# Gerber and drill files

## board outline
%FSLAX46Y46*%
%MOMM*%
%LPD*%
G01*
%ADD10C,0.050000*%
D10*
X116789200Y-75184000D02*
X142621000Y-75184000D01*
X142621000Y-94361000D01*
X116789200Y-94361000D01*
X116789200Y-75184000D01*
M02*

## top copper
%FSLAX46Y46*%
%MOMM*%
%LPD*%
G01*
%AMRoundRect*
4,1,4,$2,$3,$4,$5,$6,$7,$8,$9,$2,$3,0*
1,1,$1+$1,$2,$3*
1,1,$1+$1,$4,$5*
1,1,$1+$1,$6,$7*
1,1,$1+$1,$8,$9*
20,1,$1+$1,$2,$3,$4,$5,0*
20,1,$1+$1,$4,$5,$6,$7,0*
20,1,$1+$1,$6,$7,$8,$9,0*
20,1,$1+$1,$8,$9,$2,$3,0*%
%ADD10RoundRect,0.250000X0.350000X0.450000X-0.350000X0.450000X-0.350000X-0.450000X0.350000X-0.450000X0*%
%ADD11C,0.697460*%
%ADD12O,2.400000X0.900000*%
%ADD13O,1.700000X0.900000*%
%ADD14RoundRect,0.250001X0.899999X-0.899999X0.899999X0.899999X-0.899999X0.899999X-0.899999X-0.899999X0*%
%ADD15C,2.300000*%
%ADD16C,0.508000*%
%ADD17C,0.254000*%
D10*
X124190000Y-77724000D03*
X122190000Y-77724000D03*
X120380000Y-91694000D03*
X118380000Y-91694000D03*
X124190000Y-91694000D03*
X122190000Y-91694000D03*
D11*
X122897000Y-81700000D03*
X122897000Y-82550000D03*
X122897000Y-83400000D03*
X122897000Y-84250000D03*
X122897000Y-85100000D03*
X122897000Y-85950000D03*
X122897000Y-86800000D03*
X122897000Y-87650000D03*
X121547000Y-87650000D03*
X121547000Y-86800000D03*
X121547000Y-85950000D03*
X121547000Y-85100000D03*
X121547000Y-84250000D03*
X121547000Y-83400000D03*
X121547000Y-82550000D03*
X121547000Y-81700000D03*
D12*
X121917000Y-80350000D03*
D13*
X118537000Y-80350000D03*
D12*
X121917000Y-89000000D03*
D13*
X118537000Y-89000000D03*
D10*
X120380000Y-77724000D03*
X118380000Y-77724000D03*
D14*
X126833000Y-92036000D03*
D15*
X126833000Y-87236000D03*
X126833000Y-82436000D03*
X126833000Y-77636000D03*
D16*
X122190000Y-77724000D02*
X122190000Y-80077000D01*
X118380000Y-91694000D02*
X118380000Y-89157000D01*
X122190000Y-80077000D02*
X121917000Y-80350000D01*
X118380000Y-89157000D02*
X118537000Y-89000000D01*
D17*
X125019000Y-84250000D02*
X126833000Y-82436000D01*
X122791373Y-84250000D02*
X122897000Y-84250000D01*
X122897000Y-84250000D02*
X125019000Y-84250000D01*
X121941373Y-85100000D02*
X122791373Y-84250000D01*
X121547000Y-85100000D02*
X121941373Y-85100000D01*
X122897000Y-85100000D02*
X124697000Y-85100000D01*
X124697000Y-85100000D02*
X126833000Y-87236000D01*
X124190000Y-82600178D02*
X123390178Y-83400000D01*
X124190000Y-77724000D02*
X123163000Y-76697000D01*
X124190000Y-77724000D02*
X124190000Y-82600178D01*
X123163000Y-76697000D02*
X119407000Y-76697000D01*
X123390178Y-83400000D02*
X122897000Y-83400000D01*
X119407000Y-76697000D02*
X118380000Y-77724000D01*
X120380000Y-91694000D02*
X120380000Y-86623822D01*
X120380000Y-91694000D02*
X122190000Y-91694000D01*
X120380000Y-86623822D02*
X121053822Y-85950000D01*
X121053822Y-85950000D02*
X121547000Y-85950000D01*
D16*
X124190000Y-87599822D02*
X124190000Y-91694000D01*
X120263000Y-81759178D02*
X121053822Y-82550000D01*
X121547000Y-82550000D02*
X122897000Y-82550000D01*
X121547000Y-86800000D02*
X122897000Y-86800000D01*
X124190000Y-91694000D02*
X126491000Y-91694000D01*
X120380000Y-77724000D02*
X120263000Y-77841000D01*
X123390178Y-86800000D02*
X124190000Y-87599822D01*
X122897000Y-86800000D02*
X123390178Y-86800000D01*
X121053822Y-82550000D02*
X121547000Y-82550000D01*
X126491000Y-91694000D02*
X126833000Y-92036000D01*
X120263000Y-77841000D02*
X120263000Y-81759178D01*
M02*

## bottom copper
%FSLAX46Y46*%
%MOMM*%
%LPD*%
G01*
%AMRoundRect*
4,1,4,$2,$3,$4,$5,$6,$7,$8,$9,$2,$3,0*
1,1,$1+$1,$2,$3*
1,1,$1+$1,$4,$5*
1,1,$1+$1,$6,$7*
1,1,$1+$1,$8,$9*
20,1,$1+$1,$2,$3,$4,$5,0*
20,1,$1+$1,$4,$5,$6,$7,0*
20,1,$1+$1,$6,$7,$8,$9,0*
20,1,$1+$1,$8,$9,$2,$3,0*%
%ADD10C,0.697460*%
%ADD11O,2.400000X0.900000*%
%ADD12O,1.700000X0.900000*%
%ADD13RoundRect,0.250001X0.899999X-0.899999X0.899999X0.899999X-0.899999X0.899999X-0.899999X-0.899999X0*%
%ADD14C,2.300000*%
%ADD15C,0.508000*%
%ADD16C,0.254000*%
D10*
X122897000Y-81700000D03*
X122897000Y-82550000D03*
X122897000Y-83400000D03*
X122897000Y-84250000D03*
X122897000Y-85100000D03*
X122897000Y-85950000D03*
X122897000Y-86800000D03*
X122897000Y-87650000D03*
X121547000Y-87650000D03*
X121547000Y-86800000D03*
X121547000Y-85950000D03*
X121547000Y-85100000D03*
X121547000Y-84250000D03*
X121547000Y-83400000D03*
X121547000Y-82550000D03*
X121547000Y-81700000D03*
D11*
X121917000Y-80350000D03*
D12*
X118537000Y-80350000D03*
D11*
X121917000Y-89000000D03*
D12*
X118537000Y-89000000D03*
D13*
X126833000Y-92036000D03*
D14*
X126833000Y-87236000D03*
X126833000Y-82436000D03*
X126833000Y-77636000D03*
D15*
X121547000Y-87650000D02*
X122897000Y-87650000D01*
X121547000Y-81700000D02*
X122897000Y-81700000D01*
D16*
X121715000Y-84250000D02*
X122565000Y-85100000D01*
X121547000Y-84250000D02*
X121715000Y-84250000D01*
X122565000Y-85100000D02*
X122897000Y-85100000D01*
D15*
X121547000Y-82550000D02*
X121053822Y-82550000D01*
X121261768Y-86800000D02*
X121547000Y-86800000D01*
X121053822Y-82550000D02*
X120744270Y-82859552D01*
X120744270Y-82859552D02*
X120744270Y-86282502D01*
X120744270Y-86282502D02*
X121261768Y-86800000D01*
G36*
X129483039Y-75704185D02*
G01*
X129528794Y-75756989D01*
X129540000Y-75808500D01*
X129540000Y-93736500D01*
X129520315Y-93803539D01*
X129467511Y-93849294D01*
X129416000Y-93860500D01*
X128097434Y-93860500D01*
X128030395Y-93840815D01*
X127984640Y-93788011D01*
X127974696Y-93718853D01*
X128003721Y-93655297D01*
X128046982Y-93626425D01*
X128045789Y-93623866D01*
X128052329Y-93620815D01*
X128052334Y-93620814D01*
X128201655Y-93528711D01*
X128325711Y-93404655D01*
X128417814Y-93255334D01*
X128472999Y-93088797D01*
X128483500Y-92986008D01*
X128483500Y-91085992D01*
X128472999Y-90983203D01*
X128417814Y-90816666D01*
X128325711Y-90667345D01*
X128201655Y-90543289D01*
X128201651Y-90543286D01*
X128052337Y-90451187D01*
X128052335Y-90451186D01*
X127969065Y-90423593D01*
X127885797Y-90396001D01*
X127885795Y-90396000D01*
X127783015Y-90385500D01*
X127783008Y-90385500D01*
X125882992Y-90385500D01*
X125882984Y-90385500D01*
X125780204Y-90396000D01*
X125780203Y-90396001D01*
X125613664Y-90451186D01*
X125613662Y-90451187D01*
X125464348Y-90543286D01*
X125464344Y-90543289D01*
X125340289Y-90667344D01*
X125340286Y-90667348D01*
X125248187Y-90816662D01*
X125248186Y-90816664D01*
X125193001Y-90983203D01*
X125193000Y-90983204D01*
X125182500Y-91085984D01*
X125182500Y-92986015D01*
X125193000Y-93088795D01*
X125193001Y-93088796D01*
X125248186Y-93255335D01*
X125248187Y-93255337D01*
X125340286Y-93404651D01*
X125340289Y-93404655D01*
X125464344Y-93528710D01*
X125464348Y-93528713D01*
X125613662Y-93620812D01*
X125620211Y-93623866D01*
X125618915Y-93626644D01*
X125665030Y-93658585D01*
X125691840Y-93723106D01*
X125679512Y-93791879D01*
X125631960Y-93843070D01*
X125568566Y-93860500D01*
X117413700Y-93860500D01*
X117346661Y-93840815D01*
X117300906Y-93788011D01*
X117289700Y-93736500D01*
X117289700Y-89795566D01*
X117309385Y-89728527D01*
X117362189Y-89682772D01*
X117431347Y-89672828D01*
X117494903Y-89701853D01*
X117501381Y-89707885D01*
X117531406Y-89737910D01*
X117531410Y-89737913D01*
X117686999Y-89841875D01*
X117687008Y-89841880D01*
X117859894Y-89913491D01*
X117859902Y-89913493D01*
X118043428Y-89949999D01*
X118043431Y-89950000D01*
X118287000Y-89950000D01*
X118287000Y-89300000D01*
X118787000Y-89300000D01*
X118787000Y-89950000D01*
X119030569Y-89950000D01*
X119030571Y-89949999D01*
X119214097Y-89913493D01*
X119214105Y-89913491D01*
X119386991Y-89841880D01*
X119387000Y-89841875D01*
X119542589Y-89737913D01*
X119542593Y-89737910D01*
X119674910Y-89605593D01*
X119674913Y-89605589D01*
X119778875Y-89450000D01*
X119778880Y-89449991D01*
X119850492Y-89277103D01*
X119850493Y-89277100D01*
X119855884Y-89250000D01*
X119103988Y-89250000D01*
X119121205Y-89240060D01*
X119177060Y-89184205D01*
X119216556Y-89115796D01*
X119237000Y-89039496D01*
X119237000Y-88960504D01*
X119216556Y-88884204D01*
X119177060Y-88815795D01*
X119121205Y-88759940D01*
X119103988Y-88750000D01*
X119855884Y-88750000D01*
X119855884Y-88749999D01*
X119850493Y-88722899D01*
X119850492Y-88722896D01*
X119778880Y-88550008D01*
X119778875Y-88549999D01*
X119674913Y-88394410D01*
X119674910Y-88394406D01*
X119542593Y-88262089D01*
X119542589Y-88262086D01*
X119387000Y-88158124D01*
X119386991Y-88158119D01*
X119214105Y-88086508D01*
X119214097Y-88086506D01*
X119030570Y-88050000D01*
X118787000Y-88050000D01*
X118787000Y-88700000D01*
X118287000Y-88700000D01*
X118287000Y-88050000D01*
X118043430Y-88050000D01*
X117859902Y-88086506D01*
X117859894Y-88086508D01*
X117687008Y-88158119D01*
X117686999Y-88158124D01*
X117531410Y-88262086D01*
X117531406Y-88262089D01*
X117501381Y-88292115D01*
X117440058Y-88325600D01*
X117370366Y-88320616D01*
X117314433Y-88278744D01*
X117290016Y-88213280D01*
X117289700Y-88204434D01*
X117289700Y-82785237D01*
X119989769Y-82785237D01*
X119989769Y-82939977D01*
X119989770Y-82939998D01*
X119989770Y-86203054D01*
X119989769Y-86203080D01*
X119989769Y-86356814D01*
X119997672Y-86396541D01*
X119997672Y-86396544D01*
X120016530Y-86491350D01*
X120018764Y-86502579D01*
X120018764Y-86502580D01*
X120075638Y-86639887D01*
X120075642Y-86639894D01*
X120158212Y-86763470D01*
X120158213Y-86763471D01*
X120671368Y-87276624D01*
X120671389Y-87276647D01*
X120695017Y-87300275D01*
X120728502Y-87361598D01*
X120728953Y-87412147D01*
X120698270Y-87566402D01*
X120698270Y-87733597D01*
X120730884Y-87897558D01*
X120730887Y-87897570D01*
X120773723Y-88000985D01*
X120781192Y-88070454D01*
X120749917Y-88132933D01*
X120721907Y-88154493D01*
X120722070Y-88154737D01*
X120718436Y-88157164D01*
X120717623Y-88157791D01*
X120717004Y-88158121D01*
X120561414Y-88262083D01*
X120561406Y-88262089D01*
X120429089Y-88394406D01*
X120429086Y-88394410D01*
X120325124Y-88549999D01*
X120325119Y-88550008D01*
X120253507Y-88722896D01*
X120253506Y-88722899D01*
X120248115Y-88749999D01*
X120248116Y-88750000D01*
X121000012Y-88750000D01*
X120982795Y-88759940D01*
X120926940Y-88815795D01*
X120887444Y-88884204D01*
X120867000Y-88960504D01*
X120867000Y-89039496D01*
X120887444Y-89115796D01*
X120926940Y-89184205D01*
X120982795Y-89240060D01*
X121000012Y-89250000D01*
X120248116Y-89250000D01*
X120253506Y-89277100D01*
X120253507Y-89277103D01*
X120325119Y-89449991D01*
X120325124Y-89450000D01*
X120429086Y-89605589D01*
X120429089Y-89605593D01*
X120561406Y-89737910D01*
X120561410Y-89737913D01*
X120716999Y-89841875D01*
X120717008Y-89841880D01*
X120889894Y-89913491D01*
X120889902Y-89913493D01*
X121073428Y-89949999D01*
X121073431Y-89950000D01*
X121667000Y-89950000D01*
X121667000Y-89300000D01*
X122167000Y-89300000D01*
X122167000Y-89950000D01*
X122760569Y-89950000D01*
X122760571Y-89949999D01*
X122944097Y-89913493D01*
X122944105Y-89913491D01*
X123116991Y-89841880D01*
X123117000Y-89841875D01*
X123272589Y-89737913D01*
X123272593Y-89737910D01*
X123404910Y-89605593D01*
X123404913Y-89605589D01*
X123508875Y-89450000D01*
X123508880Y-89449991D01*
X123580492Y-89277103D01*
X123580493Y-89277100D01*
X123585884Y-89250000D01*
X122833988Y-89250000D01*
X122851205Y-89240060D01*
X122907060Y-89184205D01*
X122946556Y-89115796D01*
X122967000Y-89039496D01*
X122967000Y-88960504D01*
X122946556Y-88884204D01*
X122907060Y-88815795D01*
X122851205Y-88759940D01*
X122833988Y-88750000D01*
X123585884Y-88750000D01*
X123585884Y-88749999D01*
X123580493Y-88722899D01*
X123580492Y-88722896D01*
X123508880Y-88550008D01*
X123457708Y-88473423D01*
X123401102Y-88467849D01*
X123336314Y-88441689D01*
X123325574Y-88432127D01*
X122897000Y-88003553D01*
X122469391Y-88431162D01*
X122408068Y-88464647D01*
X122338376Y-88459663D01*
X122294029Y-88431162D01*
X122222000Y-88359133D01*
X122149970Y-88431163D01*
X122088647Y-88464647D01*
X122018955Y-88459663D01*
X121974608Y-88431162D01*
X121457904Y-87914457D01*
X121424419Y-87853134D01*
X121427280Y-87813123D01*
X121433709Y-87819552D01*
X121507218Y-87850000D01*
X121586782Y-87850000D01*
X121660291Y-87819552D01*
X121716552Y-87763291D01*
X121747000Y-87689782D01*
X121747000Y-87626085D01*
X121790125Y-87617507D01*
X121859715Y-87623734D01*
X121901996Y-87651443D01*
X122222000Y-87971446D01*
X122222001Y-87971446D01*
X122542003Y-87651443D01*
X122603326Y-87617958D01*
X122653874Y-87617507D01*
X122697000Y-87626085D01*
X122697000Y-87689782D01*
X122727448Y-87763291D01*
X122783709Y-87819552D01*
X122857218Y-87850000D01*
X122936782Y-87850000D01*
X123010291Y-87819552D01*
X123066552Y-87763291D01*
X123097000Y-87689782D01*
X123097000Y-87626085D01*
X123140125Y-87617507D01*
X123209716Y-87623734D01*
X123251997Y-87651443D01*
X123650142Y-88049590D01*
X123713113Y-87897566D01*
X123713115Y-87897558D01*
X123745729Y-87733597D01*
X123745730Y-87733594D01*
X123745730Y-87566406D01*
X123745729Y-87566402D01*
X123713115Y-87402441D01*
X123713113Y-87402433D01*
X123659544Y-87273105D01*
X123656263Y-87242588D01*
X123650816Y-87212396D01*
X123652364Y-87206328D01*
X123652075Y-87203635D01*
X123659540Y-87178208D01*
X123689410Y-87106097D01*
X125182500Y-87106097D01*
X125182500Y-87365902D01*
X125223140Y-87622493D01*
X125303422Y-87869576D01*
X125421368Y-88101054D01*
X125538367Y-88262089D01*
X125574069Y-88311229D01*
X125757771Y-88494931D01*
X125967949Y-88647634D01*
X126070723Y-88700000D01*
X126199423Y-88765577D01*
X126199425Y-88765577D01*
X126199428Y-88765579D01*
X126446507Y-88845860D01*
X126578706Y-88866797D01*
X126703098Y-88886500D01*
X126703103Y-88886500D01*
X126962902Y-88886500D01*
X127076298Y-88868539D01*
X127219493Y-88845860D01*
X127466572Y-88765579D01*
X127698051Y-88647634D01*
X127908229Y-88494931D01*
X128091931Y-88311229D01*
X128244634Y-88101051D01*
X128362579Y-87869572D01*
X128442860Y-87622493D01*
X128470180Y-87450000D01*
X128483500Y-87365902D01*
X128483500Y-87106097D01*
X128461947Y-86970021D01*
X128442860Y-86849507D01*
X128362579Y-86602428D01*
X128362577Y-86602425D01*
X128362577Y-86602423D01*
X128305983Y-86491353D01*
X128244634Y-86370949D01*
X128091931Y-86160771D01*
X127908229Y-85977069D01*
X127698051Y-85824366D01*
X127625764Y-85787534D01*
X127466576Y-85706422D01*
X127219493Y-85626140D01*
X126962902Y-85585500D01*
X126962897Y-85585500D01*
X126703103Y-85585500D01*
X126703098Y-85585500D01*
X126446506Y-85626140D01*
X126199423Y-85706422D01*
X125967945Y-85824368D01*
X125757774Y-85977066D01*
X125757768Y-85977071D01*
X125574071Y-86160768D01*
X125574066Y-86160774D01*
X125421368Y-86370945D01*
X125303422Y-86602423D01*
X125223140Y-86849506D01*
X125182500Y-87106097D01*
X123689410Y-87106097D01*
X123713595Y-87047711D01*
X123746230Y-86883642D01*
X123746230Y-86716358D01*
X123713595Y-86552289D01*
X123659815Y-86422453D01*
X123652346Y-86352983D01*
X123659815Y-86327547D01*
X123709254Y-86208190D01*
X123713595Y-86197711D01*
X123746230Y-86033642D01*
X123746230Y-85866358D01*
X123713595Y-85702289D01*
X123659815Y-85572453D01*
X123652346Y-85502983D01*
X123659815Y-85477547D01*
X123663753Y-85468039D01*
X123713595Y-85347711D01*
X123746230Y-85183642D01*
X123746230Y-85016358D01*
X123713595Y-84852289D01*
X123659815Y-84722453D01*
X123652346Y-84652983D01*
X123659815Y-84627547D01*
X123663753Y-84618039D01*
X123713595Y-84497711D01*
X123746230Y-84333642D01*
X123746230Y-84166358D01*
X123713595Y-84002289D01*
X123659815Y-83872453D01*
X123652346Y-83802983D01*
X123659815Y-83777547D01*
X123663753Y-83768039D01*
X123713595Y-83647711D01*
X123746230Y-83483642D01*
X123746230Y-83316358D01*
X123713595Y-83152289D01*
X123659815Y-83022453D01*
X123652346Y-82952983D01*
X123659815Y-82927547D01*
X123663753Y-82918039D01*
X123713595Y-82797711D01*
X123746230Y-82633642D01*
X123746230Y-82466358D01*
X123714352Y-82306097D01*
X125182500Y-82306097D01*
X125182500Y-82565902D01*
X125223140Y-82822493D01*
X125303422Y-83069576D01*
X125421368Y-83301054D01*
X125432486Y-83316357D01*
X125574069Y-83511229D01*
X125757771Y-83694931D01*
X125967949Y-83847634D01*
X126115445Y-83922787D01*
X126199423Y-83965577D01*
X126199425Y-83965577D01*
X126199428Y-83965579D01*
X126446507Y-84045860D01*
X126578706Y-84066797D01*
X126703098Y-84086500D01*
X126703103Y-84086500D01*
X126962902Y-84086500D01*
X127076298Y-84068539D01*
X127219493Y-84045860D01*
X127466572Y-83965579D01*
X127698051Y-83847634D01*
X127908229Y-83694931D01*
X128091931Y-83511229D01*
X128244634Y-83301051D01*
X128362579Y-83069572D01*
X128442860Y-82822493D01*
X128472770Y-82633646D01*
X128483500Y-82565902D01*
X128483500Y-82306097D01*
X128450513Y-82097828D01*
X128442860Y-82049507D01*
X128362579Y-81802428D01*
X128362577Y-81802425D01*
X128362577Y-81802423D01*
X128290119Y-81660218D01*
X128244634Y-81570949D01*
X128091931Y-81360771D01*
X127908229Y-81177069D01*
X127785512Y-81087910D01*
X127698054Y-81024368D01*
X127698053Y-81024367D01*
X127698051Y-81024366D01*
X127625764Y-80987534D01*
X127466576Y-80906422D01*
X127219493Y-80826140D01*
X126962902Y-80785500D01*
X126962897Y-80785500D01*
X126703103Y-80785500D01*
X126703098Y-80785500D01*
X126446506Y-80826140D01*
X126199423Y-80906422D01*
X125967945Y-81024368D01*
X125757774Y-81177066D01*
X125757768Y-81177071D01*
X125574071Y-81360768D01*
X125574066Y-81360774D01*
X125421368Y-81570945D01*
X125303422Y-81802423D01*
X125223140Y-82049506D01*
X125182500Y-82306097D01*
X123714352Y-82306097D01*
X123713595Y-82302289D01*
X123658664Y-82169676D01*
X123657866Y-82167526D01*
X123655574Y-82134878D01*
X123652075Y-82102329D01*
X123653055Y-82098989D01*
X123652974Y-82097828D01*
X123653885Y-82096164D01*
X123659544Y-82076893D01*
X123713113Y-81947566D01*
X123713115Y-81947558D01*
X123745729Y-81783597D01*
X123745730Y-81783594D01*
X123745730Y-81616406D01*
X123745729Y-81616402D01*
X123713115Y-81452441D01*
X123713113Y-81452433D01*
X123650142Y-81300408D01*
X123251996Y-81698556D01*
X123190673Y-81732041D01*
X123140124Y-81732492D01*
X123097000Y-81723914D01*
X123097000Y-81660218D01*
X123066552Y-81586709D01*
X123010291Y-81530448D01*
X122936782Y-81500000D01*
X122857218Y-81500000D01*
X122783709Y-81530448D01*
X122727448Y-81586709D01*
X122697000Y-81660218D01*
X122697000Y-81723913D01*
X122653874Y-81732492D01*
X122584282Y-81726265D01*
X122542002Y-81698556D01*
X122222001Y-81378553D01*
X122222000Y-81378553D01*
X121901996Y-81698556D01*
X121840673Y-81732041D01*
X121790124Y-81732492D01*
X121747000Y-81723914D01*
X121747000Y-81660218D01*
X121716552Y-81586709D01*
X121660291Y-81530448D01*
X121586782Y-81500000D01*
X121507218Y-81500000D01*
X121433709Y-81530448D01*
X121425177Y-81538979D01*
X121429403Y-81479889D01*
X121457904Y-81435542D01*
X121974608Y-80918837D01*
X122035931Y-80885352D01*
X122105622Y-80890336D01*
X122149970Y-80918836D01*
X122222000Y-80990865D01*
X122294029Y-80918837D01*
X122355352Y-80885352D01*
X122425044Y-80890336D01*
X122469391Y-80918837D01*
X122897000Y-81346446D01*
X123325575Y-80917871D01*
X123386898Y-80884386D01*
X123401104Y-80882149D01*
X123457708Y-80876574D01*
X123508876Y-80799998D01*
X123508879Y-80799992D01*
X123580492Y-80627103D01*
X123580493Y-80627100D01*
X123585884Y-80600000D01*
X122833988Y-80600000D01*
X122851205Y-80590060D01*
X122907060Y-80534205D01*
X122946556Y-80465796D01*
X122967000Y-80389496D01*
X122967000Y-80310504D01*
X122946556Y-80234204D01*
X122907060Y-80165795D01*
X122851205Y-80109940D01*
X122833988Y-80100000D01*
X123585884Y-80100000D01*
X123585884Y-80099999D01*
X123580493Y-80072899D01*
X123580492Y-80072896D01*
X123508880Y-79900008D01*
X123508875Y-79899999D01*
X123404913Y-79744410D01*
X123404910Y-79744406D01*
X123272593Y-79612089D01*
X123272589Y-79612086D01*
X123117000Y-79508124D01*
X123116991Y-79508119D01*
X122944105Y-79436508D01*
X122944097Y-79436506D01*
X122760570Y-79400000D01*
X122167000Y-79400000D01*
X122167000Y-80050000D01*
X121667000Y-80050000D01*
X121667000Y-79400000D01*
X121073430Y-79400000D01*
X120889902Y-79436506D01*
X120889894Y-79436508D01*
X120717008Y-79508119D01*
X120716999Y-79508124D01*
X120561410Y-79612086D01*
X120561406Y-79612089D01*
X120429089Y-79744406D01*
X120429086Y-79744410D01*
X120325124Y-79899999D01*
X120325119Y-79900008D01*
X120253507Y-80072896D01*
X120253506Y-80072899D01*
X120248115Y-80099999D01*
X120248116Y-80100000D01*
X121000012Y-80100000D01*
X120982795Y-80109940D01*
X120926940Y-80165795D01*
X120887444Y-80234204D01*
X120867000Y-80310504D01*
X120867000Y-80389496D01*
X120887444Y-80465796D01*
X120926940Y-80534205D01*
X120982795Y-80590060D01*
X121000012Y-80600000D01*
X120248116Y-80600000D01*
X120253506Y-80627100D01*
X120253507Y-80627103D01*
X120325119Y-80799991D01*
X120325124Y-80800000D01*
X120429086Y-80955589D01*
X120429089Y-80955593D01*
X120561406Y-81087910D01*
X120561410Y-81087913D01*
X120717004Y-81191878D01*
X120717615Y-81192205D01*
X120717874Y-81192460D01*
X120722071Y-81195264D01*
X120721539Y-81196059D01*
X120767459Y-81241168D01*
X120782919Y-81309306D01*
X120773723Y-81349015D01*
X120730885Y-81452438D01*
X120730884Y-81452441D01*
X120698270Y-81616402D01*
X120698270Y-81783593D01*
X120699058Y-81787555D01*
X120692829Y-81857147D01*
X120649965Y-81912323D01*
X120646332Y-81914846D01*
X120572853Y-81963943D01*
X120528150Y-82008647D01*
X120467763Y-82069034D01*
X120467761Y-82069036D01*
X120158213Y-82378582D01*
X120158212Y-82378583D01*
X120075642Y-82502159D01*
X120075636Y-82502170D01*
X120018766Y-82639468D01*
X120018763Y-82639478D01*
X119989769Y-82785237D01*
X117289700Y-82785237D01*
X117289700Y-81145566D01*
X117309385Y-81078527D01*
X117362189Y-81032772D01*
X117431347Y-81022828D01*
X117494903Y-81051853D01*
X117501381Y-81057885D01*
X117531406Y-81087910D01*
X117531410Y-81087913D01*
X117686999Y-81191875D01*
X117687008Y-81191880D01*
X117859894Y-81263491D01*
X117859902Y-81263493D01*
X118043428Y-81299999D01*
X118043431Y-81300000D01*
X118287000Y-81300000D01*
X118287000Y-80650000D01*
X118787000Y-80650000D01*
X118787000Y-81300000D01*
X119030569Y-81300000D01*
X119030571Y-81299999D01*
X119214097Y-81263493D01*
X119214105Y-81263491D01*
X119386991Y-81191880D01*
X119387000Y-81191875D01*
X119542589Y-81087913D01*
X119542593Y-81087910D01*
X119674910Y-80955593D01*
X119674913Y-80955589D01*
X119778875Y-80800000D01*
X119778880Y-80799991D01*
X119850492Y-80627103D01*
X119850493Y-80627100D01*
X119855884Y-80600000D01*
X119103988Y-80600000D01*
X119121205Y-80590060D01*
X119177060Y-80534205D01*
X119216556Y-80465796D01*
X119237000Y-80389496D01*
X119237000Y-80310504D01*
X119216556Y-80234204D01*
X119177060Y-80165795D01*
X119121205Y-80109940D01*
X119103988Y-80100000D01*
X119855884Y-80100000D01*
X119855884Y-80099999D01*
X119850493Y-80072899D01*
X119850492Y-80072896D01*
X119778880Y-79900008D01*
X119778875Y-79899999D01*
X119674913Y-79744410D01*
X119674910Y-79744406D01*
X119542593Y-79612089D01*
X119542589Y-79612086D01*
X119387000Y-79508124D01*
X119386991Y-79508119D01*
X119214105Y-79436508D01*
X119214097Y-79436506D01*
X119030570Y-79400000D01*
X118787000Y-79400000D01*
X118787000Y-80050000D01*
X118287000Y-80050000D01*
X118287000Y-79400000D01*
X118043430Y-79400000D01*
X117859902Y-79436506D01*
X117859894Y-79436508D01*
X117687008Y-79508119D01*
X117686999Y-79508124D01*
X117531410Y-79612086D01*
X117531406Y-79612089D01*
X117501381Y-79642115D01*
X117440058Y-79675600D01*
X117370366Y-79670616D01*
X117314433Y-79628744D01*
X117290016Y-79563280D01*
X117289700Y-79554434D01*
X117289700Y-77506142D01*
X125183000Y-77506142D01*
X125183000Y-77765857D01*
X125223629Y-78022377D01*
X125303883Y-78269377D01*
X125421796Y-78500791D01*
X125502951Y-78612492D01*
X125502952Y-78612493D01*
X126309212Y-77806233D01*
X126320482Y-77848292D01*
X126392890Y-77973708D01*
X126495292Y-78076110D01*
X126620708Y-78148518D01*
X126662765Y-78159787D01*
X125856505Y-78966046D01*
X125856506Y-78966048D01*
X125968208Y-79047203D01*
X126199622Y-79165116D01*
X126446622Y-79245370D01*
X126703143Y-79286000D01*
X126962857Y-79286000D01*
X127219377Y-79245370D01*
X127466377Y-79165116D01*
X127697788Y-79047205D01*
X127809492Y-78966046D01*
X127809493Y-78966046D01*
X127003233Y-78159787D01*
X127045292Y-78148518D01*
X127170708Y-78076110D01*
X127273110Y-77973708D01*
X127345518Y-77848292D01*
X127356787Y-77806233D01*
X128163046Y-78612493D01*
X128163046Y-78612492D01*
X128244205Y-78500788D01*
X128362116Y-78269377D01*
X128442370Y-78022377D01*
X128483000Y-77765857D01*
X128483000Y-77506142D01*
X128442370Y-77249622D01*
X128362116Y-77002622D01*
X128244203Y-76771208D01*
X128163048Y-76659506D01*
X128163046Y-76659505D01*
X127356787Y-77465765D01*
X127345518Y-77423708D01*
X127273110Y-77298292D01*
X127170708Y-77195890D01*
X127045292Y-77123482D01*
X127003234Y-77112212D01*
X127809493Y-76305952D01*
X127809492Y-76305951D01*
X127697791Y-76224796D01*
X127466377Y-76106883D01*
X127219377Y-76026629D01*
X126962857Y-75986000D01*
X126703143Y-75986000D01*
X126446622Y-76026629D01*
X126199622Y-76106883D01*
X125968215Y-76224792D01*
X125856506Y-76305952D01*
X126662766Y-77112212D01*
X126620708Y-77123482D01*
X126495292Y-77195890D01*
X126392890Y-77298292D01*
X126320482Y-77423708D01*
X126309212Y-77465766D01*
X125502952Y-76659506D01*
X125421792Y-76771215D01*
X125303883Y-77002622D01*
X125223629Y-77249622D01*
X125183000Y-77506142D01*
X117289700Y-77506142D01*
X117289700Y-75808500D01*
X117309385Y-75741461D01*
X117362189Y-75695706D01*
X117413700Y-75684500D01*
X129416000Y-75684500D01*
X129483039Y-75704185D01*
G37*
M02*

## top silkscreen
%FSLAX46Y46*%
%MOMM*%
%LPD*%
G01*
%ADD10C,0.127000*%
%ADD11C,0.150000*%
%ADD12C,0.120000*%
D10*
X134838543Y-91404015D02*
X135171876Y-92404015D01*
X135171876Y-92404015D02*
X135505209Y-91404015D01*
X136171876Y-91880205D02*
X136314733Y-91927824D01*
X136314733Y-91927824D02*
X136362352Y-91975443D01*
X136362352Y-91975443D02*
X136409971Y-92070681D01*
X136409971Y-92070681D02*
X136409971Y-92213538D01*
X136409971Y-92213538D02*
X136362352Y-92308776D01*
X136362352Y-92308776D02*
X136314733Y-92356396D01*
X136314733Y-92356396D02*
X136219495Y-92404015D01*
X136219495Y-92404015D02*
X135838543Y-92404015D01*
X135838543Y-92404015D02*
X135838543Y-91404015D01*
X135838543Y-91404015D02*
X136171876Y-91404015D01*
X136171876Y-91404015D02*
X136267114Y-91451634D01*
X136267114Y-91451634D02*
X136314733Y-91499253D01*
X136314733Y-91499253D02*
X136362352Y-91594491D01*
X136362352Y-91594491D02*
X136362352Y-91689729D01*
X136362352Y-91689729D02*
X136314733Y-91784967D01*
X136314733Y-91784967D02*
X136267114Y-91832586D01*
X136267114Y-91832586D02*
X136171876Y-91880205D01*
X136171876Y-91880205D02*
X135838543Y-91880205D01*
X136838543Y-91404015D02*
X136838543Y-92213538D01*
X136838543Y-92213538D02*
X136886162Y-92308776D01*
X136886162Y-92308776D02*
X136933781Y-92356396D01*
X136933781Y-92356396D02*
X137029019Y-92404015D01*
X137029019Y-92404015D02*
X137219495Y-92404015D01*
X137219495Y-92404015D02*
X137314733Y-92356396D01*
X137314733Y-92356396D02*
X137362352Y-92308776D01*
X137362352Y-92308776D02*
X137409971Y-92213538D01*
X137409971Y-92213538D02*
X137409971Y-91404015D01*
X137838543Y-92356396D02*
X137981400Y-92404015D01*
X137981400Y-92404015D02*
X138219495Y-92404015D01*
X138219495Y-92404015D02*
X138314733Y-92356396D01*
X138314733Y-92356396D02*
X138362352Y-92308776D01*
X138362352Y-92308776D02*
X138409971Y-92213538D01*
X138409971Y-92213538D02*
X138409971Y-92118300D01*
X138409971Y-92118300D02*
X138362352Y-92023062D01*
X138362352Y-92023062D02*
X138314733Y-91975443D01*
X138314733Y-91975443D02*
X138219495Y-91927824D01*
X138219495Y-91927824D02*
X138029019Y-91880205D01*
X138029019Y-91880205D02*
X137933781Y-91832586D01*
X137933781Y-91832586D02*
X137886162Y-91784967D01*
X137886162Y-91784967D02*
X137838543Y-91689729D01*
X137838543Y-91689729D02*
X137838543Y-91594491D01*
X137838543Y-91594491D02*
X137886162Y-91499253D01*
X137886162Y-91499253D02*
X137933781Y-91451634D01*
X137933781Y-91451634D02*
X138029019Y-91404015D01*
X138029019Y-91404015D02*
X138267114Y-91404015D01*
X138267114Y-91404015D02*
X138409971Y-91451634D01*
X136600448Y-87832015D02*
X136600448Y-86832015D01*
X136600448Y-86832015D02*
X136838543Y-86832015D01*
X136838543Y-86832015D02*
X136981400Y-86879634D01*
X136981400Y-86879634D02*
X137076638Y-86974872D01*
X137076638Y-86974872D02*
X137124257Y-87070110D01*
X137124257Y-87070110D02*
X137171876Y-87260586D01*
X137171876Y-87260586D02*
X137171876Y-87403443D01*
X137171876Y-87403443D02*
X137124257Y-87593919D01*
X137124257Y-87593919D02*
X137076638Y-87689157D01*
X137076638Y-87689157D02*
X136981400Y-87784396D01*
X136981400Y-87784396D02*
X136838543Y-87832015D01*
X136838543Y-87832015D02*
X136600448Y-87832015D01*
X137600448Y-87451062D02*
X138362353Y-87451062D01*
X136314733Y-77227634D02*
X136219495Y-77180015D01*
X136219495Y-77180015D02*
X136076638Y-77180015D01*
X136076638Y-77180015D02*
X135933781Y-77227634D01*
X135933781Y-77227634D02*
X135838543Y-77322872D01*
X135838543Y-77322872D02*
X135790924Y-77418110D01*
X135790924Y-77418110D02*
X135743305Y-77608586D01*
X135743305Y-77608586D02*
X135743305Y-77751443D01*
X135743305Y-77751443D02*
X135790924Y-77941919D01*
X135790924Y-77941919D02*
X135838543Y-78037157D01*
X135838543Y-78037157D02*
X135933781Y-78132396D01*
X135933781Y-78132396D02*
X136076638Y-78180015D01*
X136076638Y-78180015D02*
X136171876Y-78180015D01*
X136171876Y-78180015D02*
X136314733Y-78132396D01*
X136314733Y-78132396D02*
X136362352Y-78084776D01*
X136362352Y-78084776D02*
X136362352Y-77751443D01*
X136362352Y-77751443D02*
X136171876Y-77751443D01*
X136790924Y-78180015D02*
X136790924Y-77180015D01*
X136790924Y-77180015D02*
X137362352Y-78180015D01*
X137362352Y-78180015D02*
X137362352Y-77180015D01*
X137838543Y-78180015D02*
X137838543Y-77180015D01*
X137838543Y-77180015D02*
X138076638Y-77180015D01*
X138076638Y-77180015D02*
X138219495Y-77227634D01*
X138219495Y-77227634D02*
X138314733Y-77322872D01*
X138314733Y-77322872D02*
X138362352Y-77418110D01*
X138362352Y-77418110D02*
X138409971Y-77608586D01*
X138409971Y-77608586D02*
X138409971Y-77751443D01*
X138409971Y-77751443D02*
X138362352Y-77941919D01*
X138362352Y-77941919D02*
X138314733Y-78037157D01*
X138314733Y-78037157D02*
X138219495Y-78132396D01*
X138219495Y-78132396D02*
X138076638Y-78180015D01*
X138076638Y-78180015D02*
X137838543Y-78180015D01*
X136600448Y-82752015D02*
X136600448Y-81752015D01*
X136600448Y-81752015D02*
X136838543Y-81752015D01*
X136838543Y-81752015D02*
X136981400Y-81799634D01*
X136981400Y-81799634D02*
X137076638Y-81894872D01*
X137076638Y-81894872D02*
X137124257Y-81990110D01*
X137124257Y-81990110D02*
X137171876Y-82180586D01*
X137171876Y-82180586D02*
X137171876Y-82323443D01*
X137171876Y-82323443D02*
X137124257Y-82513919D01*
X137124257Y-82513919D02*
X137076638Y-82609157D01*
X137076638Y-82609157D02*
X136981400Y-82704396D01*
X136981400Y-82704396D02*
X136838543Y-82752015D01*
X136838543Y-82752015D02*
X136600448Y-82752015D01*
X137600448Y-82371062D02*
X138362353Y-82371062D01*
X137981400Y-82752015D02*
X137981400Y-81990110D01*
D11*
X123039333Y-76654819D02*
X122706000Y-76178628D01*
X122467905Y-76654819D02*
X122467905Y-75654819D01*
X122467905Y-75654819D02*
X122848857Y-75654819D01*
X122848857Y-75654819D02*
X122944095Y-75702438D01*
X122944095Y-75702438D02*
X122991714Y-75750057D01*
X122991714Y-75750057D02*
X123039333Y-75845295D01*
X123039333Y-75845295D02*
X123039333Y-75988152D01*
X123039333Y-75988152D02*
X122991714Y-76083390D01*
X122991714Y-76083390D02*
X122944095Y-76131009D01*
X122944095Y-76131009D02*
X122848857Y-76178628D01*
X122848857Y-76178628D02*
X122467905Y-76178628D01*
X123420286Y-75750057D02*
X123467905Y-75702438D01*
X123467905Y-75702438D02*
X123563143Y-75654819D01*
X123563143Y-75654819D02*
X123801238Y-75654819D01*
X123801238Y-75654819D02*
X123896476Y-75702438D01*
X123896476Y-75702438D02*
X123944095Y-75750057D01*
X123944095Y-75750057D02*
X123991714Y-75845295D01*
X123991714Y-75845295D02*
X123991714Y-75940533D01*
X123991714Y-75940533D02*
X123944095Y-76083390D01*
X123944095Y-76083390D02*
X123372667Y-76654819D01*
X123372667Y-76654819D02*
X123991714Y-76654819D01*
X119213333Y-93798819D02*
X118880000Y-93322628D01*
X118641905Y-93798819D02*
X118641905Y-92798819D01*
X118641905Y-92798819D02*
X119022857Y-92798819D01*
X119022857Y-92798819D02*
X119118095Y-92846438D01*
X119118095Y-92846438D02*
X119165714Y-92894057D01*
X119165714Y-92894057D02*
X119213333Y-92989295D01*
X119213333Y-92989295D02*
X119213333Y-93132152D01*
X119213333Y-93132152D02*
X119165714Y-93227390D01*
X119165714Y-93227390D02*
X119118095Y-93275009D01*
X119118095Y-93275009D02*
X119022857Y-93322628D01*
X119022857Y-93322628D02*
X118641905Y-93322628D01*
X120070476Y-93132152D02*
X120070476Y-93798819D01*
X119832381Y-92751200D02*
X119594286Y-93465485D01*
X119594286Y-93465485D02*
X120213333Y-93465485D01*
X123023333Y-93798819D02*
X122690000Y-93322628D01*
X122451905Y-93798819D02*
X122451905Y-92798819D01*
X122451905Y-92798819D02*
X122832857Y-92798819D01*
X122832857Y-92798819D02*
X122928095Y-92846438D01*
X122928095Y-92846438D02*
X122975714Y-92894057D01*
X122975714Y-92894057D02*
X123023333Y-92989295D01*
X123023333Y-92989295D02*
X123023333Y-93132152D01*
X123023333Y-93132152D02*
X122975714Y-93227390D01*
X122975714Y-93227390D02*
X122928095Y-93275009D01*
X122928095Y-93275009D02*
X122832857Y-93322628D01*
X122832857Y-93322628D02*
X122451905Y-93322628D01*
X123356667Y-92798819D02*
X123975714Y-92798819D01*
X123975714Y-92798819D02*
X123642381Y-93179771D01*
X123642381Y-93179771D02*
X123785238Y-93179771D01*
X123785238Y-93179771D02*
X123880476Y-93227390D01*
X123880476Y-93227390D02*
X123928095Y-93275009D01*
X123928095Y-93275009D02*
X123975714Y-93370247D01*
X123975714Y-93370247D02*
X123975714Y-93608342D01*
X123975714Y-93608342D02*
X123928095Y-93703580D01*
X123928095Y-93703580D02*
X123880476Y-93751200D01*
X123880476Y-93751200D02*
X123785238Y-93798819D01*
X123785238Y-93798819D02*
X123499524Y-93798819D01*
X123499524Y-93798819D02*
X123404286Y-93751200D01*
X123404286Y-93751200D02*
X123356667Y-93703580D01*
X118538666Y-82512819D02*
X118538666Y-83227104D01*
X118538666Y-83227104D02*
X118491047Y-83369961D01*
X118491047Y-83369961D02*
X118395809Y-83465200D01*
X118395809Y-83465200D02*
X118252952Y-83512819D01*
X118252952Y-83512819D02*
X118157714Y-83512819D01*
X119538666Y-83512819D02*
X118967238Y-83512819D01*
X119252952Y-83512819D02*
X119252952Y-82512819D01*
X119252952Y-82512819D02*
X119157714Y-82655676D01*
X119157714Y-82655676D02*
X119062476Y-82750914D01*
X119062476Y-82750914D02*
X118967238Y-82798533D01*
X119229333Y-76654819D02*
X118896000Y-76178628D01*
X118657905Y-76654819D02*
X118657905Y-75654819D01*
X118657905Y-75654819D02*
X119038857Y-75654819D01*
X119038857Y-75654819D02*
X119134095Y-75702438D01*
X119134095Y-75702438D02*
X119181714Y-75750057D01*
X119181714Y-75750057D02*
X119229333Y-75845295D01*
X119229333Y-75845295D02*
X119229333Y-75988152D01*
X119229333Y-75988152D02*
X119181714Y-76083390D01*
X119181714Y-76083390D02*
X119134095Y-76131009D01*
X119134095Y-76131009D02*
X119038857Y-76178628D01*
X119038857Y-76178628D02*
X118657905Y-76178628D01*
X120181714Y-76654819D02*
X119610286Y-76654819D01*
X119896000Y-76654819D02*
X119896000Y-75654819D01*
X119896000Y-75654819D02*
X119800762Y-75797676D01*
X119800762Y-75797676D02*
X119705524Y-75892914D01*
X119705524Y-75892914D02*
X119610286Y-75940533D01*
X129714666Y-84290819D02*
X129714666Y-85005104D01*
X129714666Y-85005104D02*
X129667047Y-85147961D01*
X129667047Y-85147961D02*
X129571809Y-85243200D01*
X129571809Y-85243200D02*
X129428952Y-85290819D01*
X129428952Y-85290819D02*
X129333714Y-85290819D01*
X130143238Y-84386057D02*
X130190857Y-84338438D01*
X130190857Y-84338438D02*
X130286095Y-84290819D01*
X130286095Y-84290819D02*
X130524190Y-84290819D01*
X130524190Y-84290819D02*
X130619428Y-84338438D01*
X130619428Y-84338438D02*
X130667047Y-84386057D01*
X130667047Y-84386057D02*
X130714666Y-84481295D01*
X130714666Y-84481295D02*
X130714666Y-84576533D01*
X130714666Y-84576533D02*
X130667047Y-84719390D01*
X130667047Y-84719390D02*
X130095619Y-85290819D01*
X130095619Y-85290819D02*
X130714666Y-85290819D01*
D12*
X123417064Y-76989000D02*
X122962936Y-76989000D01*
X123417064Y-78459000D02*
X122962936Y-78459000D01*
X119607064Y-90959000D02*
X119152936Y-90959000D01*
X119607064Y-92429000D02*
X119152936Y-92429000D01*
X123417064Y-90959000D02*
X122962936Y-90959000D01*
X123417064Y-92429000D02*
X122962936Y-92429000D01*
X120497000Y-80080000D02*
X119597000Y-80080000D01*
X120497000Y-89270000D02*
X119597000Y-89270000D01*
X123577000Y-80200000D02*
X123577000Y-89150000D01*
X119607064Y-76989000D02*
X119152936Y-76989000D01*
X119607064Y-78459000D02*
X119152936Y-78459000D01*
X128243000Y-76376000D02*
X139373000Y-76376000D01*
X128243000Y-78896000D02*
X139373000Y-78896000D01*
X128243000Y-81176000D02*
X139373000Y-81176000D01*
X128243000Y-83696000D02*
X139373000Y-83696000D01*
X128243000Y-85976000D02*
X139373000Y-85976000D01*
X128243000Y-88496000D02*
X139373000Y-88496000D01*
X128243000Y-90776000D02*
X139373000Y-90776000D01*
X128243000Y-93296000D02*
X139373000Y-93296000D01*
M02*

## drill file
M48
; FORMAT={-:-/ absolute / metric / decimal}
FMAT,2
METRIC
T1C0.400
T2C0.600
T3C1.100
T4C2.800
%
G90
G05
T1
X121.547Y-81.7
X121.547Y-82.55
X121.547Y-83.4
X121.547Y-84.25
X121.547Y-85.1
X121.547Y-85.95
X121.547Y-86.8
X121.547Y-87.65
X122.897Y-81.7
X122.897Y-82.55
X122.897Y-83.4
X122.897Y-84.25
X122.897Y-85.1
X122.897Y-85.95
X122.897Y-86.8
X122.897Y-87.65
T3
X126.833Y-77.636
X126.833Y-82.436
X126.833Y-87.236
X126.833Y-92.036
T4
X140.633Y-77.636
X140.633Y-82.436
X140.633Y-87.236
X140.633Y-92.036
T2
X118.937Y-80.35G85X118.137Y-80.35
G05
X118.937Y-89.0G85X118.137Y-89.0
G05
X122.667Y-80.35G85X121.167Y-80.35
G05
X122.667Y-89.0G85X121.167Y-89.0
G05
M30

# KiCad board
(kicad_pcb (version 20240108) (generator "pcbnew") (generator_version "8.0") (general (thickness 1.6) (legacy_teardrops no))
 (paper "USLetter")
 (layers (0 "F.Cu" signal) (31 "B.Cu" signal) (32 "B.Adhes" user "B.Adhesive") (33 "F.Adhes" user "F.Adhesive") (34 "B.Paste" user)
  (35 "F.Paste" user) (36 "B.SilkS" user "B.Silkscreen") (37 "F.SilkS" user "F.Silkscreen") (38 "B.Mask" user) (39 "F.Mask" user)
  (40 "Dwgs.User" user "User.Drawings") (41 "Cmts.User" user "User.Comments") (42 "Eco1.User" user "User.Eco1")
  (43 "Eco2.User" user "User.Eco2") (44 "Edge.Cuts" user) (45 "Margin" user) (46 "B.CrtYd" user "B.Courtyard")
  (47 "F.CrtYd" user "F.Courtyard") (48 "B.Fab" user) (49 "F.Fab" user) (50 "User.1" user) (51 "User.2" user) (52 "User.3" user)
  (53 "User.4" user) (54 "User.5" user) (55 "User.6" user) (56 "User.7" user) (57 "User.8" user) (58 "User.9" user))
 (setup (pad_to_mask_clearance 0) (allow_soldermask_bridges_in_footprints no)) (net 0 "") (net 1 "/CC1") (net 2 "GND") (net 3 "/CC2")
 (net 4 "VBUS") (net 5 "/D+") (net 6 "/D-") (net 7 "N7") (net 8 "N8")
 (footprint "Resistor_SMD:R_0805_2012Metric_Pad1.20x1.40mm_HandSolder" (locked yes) (layer "F.Cu") (at 123.19 77.724 180)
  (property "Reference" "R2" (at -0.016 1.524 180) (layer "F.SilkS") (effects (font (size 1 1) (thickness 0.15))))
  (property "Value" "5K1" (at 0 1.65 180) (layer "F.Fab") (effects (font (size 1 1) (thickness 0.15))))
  (fp_line (start -0.227064 0.735) (end 0.227064 0.735) (stroke (width 0.12) (type solid)) (layer "F.SilkS"))
  (fp_line (start -0.227064 -0.735) (end 0.227064 -0.735) (stroke (width 0.12) (type solid)) (layer "F.SilkS"))
  (pad "1" smd roundrect (at -1 0 180) (size 1.2 1.4) (layers "F.Cu" "F.Paste" "F.Mask") (roundrect_rratio 0.208333) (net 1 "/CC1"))
  (pad "2" smd roundrect (at 1 0 180) (size 1.2 1.4) (layers "F.Cu" "F.Paste" "F.Mask") (roundrect_rratio 0.208333) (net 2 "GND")))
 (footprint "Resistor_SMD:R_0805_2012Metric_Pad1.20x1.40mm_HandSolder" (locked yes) (layer "F.Cu") (at 119.38 91.694 180)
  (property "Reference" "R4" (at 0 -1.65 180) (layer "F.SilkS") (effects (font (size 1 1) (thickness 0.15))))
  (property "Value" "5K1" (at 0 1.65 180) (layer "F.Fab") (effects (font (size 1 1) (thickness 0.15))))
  (fp_line (start -0.227064 0.735) (end 0.227064 0.735) (stroke (width 0.12) (type solid)) (layer "F.SilkS"))
  (fp_line (start -0.227064 -0.735) (end 0.227064 -0.735) (stroke (width 0.12) (type solid)) (layer "F.SilkS"))
  (pad "1" smd roundrect (at -1 0 180) (size 1.2 1.4) (layers "F.Cu" "F.Paste" "F.Mask") (roundrect_rratio 0.208333) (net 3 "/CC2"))
  (pad "2" smd roundrect (at 1 0 180) (size 1.2 1.4) (layers "F.Cu" "F.Paste" "F.Mask") (roundrect_rratio 0.208333) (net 2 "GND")))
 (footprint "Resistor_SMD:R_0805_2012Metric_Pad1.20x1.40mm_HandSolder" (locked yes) (layer "F.Cu") (at 123.19 91.694 180)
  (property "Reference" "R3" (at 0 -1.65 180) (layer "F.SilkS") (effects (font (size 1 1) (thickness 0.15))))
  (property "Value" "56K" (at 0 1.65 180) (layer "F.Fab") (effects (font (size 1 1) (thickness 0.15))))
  (fp_line (start -0.227064 0.735) (end 0.227064 0.735) (stroke (width 0.12) (type solid)) (layer "F.SilkS"))
  (fp_line (start -0.227064 -0.735) (end 0.227064 -0.735) (stroke (width 0.12) (type solid)) (layer "F.SilkS"))
  (pad "1" smd roundrect (at -1 0 180) (size 1.2 1.4) (layers "F.Cu" "F.Paste" "F.Mask") (roundrect_rratio 0.208333) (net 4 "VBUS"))
  (pad "2" smd roundrect (at 1 0 180) (size 1.2 1.4) (layers "F.Cu" "F.Paste" "F.Mask") (roundrect_rratio 0.208333) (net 3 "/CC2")))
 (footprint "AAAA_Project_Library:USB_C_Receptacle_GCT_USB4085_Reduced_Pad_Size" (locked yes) (layer "F.Cu") (at 122.897 81.7 -90)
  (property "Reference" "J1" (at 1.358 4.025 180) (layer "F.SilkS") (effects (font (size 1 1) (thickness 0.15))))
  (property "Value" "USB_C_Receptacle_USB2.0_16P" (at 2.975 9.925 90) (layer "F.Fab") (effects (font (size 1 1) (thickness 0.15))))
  (fp_line (start -1.62 2.4) (end -1.62 3.3) (stroke (width 0.12) (type solid)) (layer "F.SilkS"))
  (fp_line (start 7.57 2.4) (end 7.57 3.3) (stroke (width 0.12) (type solid)) (layer "F.SilkS"))
  (fp_line (start -1.5 -0.68) (end 7.45 -0.68) (stroke (width 0.12) (type solid)) (layer "F.SilkS"))
  (pad "A1" thru_hole circle (at 0 0 270) (size 0.69746 0.69746) (drill 0.4) (layers "*.Cu" "*.Mask") (remove_unused_layers no)
   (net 2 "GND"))
  (pad "A4" thru_hole circle (at 0.85 0 270) (size 0.69746 0.69746) (drill 0.4) (layers "*.Cu" "*.Mask") (remove_unused_layers no)
   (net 4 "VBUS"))
  (pad "A5" thru_hole circle (at 1.7 0 270) (size 0.69746 0.69746) (drill 0.4) (layers "*.Cu" "*.Mask") (remove_unused_layers no)
   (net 1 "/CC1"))
  (pad "A6" thru_hole circle (at 2.55 0 270) (size 0.69746 0.69746) (drill 0.4) (layers "*.Cu" "*.Mask") (remove_unused_layers no)
   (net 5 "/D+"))
  (pad "A7" thru_hole circle (at 3.4 0 270) (size 0.69746 0.69746) (drill 0.4) (layers "*.Cu" "*.Mask") (remove_unused_layers no)
   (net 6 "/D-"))
  (pad "A8" thru_hole circle (at 4.25 0 270) (size 0.69746 0.69746) (drill 0.4) (layers "*.Cu" "*.Mask") (remove_unused_layers no)
   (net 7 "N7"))
  (pad "A9" thru_hole circle (at 5.1 0 270) (size 0.69746 0.69746) (drill 0.4) (layers "*.Cu" "*.Mask") (remove_unused_layers no)
   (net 4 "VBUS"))
  (pad "A12" thru_hole circle (at 5.95 0 270) (size 0.69746 0.69746) (drill 0.4) (layers "*.Cu" "*.Mask") (remove_unused_layers no)
   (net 2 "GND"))
  (pad "B1" thru_hole circle (at 5.95 1.35 270) (size 0.69746 0.69746) (drill 0.4) (layers "*.Cu" "*.Mask") (remove_unused_layers no)
   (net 2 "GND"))
  (pad "B4" thru_hole circle (at 5.1 1.35 270) (size 0.69746 0.69746) (drill 0.4) (layers "*.Cu" "*.Mask") (remove_unused_layers no)
   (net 4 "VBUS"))
  (pad "B5" thru_hole circle (at 4.25 1.35 270) (size 0.69746 0.69746) (drill 0.4) (layers "*.Cu" "*.Mask") (remove_unused_layers no)
   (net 3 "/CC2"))
  (pad "B6" thru_hole circle (at 3.4 1.35 270) (size 0.69746 0.69746) (drill 0.4) (layers "*.Cu" "*.Mask") (remove_unused_layers no)
   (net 5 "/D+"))
  (pad "B7" thru_hole circle (at 2.55 1.35 270) (size 0.69746 0.69746) (drill 0.4) (layers "*.Cu" "*.Mask") (remove_unused_layers no)
   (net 6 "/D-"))
  (pad "B8" thru_hole circle (at 1.7 1.35 270) (size 0.69746 0.69746) (drill 0.4) (layers "*.Cu" "*.Mask") (remove_unused_layers no)
   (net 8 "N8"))
  (pad "B9" thru_hole circle (at 0.85 1.35 270) (size 0.69746 0.69746) (drill 0.4) (layers "*.Cu" "*.Mask") (remove_unused_layers no)
   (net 4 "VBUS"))
  (pad "B12" thru_hole circle (at 0 1.35 270) (size 0.69746 0.69746) (drill 0.4) (layers "*.Cu" "*.Mask") (remove_unused_layers no)
   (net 2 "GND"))
  (pad "S1" thru_hole oval (at -1.35 0.98 270) (size 0.9 2.4) (drill oval 0.6 2.1) (layers "*.Cu" "*.Mask") (remove_unused_layers no)
   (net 2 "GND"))
  (pad "S1" thru_hole oval (at -1.35 4.36 270) (size 0.9 1.7) (drill oval 0.6 1.4) (layers "*.Cu" "*.Mask") (remove_unused_layers no)
   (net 2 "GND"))
  (pad "S1" thru_hole oval (at 7.3 0.98 270) (size 0.9 2.4) (drill oval 0.6 2.1) (layers "*.Cu" "*.Mask") (remove_unused_layers no)
   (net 2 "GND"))
  (pad "S1" thru_hole oval (at 7.3 4.36 270) (size 0.9 1.7) (drill oval 0.6 1.4) (layers "*.Cu" "*.Mask") (remove_unused_layers no)
   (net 2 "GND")))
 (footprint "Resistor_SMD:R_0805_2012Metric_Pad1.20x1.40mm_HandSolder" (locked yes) (layer "F.Cu") (at 119.38 77.724 180)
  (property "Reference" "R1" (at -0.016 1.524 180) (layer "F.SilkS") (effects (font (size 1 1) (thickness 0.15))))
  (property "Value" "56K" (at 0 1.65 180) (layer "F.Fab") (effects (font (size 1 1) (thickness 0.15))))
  (fp_line (start -0.227064 0.735) (end 0.227064 0.735) (stroke (width 0.12) (type solid)) (layer "F.SilkS"))
  (fp_line (start -0.227064 -0.735) (end 0.227064 -0.735) (stroke (width 0.12) (type solid)) (layer "F.SilkS"))
  (pad "1" smd roundrect (at -1 0 180) (size 1.2 1.4) (layers "F.Cu" "F.Paste" "F.Mask") (roundrect_rratio 0.208333) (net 4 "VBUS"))
  (pad "2" smd roundrect (at 1 0 180) (size 1.2 1.4) (layers "F.Cu" "F.Paste" "F.Mask") (roundrect_rratio 0.208333) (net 1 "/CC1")))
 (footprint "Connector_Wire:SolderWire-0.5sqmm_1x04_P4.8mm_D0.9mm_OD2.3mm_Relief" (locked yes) (layer "F.Cu") (at 126.833 92.036 90)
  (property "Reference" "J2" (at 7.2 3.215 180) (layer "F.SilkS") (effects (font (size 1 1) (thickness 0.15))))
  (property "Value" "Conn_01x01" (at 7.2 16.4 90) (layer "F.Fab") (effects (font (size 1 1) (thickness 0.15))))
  (fp_line (start 15.66 1.41) (end 15.66 12.54) (stroke (width 0.12) (type solid)) (layer "F.SilkS"))
  (fp_line (start 13.14 1.41) (end 13.14 12.54) (stroke (width 0.12) (type solid)) (layer "F.SilkS"))
  (fp_line (start 10.86 1.41) (end 10.86 12.54) (stroke (width 0.12) (type solid)) (layer "F.SilkS"))
  (fp_line (start 8.34 1.41) (end 8.34 12.54) (stroke (width 0.12) (type solid)) (layer "F.SilkS"))
  (fp_line (start 6.06 1.41) (end 6.06 12.54) (stroke (width 0.12) (type solid)) (layer "F.SilkS"))
  (fp_line (start 3.54 1.41) (end 3.54 12.54) (stroke (width 0.12) (type solid)) (layer "F.SilkS"))
  (fp_line (start 1.26 1.41) (end 1.26 12.54) (stroke (width 0.12) (type solid)) (layer "F.SilkS"))
  (fp_line (start -1.26 1.41) (end -1.26 12.54) (stroke (width 0.12) (type solid)) (layer "F.SilkS"))
  (pad "" np_thru_hole circle (at 0 13.8 90) (size 2.8 2.8) (drill 2.8) (layers "*.Cu" "*.Mask"))
  (pad "" np_thru_hole circle (at 4.8 13.8 90) (size 2.8 2.8) (drill 2.8) (layers "*.Cu" "*.Mask"))
  (pad "" np_thru_hole circle (at 9.6 13.8 90) (size 2.8 2.8) (drill 2.8) (layers "*.Cu" "*.Mask"))
  (pad "" np_thru_hole circle (at 14.4 13.8 90) (size 2.8 2.8) (drill 2.8) (layers "*.Cu" "*.Mask"))
  (pad "1" thru_hole roundrect (at 0 0 90) (size 2.3 2.3) (drill 1.1) (layers "*.Cu" "*.Mask") (remove_unused_layers no)
   (roundrect_rratio 0.108696) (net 4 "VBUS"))
  (pad "2" thru_hole circle (at 4.8 0 90) (size 2.3 2.3) (drill 1.1) (layers "*.Cu" "*.Mask") (remove_unused_layers no) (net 6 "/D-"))
  (pad "3" thru_hole circle (at 9.6 0 90) (size 2.3 2.3) (drill 1.1) (layers "*.Cu" "*.Mask") (remove_unused_layers no) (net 5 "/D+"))
  (pad "4" thru_hole circle (at 14.4 0 90) (size 2.3 2.3) (drill 1.1) (layers "*.Cu" "*.Mask") (remove_unused_layers no) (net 2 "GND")))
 (gr_rect (start 116.7892 75.184) (end 142.621 94.361) (locked yes) (stroke (width 0.05) (type default)) (fill none) (layer "Edge.Cuts"))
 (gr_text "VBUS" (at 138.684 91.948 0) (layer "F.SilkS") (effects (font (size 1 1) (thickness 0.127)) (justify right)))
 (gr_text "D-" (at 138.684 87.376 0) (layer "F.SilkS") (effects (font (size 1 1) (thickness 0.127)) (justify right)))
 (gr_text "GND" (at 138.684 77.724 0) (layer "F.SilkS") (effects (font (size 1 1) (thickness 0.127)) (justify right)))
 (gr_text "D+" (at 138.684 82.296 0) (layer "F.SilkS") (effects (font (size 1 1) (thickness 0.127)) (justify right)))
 (segment (start 122.19 77.724) (end 122.19 80.077) (width 0.508) (layer "F.Cu") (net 2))
 (segment (start 118.38 91.694) (end 118.38 89.157) (width 0.508) (layer "F.Cu") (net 2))
 (segment (start 122.19 80.077) (end 121.917 80.35) (width 0.508) (layer "F.Cu") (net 2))
 (segment (start 118.38 89.157) (end 118.537 89) (width 0.508) (layer "F.Cu") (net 2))
 (segment (start 121.547 87.65) (end 122.897 87.65) (width 0.508) (layer "B.Cu") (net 2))
 (segment (start 121.547 81.7) (end 122.897 81.7) (width 0.508) (layer "B.Cu") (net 2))
 (segment (start 125.019 84.25) (end 126.833 82.436) (width 0.254) (layer "F.Cu") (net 5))
 (segment (start 122.791373 84.25) (end 122.897 84.25) (width 0.254) (locked yes) (layer "F.Cu") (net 5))
 (segment (start 122.897 84.25) (end 125.019 84.25) (width 0.254) (layer "F.Cu") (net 5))
 (segment (start 121.941373 85.1) (end 122.791373 84.25) (width 0.254) (locked yes) (layer "F.Cu") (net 5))
 (segment (start 121.547 85.1) (end 121.941373 85.1) (width 0.254) (locked yes) (layer "F.Cu") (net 5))
 (segment (start 122.897 85.1) (end 124.697 85.1) (width 0.254) (layer "F.Cu") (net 6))
 (segment (start 124.697 85.1) (end 126.833 87.236) (width 0.254) (layer "F.Cu") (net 6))
 (segment (start 121.715 84.25) (end 122.565 85.1) (width 0.254) (locked yes) (layer "B.Cu") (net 6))
 (segment (start 121.547 84.25) (end 121.715 84.25) (width 0.254) (locked yes) (layer "B.Cu") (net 6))
 (segment (start 122.565 85.1) (end 122.897 85.1) (width 0.254) (locked yes) (layer "B.Cu") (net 6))
 (segment (start 124.19 82.600178) (end 123.390178 83.4) (width 0.254) (layer "F.Cu") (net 1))
 (segment (start 124.19 77.724) (end 123.163 76.697) (width 0.254) (layer "F.Cu") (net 1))
 (segment (start 124.19 77.724) (end 124.19 82.600178) (width 0.254) (layer "F.Cu") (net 1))
 (segment (start 123.163 76.697) (end 119.407 76.697) (width 0.254) (layer "F.Cu") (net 1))
 (segment (start 123.390178 83.4) (end 122.897 83.4) (width 0.254) (layer "F.Cu") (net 1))
 (segment (start 119.407 76.697) (end 118.38 77.724) (width 0.254) (layer "F.Cu") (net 1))
 (segment (start 120.38 91.694) (end 120.38 86.623822) (width 0.254) (layer "F.Cu") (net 3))
 (segment (start 120.38 91.694) (end 122.19 91.694) (width 0.254) (layer "F.Cu") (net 3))
 (segment (start 120.38 86.623822) (end 121.053822 85.95) (width 0.254) (layer "F.Cu") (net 3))
 (segment (start 121.053822 85.95) (end 121.547 85.95) (width 0.254) (layer "F.Cu") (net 3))
 (segment (start 124.19 87.599822) (end 124.19 91.694) (width 0.508) (layer "F.Cu") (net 4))
 (segment (start 120.263 81.759178) (end 121.053822 82.55) (width 0.508) (layer "F.Cu") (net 4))
 (segment (start 121.547 82.55) (end 122.897 82.55) (width 0.508) (locked yes) (layer "F.Cu") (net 4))
 (segment (start 121.547 86.8) (end 122.897 86.8) (width 0.508) (locked yes) (layer "F.Cu") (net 4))
 (segment (start 124.19 91.694) (end 126.491 91.694) (width 0.508) (layer "F.Cu") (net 4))
 (segment (start 120.38 77.724) (end 120.263 77.841) (width 0.508) (layer "F.Cu") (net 4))
 (segment (start 123.390178 86.8) (end 124.19 87.599822) (width 0.508) (layer "F.Cu") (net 4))
 (segment (start 122.897 86.8) (end 123.390178 86.8) (width 0.508) (layer "F.Cu") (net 4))
 (segment (start 121.053822 82.55) (end 121.547 82.55) (width 0.508) (layer "F.Cu") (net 4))
 (segment (start 126.491 91.694) (end 126.833 92.036) (width 0.508) (layer "F.Cu") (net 4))
 (segment (start 120.263 77.841) (end 120.263 81.759178) (width 0.508) (layer "F.Cu") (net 4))
 (segment (start 121.547 82.55) (end 121.053822 82.55) (width 0.508) (locked yes) (layer "B.Cu") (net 4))
 (segment (start 121.261768 86.8) (end 121.547 86.8) (width 0.508) (locked yes) (layer "B.Cu") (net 4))
 (segment (start 121.053822 82.55) (end 120.74427 82.859552) (width 0.508) (locked yes) (layer "B.Cu") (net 4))
 (segment (start 120.74427 82.859552) (end 120.74427 86.282502) (width 0.508) (locked yes) (layer "B.Cu") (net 4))
 (segment (start 120.74427 86.282502) (end 121.261768 86.8) (width 0.508) (locked yes) (layer "B.Cu") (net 4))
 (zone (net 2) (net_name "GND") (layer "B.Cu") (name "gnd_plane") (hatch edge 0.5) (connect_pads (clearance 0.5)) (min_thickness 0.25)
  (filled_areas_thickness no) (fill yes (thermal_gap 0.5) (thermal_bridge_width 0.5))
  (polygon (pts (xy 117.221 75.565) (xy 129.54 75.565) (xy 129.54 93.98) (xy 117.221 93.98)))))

